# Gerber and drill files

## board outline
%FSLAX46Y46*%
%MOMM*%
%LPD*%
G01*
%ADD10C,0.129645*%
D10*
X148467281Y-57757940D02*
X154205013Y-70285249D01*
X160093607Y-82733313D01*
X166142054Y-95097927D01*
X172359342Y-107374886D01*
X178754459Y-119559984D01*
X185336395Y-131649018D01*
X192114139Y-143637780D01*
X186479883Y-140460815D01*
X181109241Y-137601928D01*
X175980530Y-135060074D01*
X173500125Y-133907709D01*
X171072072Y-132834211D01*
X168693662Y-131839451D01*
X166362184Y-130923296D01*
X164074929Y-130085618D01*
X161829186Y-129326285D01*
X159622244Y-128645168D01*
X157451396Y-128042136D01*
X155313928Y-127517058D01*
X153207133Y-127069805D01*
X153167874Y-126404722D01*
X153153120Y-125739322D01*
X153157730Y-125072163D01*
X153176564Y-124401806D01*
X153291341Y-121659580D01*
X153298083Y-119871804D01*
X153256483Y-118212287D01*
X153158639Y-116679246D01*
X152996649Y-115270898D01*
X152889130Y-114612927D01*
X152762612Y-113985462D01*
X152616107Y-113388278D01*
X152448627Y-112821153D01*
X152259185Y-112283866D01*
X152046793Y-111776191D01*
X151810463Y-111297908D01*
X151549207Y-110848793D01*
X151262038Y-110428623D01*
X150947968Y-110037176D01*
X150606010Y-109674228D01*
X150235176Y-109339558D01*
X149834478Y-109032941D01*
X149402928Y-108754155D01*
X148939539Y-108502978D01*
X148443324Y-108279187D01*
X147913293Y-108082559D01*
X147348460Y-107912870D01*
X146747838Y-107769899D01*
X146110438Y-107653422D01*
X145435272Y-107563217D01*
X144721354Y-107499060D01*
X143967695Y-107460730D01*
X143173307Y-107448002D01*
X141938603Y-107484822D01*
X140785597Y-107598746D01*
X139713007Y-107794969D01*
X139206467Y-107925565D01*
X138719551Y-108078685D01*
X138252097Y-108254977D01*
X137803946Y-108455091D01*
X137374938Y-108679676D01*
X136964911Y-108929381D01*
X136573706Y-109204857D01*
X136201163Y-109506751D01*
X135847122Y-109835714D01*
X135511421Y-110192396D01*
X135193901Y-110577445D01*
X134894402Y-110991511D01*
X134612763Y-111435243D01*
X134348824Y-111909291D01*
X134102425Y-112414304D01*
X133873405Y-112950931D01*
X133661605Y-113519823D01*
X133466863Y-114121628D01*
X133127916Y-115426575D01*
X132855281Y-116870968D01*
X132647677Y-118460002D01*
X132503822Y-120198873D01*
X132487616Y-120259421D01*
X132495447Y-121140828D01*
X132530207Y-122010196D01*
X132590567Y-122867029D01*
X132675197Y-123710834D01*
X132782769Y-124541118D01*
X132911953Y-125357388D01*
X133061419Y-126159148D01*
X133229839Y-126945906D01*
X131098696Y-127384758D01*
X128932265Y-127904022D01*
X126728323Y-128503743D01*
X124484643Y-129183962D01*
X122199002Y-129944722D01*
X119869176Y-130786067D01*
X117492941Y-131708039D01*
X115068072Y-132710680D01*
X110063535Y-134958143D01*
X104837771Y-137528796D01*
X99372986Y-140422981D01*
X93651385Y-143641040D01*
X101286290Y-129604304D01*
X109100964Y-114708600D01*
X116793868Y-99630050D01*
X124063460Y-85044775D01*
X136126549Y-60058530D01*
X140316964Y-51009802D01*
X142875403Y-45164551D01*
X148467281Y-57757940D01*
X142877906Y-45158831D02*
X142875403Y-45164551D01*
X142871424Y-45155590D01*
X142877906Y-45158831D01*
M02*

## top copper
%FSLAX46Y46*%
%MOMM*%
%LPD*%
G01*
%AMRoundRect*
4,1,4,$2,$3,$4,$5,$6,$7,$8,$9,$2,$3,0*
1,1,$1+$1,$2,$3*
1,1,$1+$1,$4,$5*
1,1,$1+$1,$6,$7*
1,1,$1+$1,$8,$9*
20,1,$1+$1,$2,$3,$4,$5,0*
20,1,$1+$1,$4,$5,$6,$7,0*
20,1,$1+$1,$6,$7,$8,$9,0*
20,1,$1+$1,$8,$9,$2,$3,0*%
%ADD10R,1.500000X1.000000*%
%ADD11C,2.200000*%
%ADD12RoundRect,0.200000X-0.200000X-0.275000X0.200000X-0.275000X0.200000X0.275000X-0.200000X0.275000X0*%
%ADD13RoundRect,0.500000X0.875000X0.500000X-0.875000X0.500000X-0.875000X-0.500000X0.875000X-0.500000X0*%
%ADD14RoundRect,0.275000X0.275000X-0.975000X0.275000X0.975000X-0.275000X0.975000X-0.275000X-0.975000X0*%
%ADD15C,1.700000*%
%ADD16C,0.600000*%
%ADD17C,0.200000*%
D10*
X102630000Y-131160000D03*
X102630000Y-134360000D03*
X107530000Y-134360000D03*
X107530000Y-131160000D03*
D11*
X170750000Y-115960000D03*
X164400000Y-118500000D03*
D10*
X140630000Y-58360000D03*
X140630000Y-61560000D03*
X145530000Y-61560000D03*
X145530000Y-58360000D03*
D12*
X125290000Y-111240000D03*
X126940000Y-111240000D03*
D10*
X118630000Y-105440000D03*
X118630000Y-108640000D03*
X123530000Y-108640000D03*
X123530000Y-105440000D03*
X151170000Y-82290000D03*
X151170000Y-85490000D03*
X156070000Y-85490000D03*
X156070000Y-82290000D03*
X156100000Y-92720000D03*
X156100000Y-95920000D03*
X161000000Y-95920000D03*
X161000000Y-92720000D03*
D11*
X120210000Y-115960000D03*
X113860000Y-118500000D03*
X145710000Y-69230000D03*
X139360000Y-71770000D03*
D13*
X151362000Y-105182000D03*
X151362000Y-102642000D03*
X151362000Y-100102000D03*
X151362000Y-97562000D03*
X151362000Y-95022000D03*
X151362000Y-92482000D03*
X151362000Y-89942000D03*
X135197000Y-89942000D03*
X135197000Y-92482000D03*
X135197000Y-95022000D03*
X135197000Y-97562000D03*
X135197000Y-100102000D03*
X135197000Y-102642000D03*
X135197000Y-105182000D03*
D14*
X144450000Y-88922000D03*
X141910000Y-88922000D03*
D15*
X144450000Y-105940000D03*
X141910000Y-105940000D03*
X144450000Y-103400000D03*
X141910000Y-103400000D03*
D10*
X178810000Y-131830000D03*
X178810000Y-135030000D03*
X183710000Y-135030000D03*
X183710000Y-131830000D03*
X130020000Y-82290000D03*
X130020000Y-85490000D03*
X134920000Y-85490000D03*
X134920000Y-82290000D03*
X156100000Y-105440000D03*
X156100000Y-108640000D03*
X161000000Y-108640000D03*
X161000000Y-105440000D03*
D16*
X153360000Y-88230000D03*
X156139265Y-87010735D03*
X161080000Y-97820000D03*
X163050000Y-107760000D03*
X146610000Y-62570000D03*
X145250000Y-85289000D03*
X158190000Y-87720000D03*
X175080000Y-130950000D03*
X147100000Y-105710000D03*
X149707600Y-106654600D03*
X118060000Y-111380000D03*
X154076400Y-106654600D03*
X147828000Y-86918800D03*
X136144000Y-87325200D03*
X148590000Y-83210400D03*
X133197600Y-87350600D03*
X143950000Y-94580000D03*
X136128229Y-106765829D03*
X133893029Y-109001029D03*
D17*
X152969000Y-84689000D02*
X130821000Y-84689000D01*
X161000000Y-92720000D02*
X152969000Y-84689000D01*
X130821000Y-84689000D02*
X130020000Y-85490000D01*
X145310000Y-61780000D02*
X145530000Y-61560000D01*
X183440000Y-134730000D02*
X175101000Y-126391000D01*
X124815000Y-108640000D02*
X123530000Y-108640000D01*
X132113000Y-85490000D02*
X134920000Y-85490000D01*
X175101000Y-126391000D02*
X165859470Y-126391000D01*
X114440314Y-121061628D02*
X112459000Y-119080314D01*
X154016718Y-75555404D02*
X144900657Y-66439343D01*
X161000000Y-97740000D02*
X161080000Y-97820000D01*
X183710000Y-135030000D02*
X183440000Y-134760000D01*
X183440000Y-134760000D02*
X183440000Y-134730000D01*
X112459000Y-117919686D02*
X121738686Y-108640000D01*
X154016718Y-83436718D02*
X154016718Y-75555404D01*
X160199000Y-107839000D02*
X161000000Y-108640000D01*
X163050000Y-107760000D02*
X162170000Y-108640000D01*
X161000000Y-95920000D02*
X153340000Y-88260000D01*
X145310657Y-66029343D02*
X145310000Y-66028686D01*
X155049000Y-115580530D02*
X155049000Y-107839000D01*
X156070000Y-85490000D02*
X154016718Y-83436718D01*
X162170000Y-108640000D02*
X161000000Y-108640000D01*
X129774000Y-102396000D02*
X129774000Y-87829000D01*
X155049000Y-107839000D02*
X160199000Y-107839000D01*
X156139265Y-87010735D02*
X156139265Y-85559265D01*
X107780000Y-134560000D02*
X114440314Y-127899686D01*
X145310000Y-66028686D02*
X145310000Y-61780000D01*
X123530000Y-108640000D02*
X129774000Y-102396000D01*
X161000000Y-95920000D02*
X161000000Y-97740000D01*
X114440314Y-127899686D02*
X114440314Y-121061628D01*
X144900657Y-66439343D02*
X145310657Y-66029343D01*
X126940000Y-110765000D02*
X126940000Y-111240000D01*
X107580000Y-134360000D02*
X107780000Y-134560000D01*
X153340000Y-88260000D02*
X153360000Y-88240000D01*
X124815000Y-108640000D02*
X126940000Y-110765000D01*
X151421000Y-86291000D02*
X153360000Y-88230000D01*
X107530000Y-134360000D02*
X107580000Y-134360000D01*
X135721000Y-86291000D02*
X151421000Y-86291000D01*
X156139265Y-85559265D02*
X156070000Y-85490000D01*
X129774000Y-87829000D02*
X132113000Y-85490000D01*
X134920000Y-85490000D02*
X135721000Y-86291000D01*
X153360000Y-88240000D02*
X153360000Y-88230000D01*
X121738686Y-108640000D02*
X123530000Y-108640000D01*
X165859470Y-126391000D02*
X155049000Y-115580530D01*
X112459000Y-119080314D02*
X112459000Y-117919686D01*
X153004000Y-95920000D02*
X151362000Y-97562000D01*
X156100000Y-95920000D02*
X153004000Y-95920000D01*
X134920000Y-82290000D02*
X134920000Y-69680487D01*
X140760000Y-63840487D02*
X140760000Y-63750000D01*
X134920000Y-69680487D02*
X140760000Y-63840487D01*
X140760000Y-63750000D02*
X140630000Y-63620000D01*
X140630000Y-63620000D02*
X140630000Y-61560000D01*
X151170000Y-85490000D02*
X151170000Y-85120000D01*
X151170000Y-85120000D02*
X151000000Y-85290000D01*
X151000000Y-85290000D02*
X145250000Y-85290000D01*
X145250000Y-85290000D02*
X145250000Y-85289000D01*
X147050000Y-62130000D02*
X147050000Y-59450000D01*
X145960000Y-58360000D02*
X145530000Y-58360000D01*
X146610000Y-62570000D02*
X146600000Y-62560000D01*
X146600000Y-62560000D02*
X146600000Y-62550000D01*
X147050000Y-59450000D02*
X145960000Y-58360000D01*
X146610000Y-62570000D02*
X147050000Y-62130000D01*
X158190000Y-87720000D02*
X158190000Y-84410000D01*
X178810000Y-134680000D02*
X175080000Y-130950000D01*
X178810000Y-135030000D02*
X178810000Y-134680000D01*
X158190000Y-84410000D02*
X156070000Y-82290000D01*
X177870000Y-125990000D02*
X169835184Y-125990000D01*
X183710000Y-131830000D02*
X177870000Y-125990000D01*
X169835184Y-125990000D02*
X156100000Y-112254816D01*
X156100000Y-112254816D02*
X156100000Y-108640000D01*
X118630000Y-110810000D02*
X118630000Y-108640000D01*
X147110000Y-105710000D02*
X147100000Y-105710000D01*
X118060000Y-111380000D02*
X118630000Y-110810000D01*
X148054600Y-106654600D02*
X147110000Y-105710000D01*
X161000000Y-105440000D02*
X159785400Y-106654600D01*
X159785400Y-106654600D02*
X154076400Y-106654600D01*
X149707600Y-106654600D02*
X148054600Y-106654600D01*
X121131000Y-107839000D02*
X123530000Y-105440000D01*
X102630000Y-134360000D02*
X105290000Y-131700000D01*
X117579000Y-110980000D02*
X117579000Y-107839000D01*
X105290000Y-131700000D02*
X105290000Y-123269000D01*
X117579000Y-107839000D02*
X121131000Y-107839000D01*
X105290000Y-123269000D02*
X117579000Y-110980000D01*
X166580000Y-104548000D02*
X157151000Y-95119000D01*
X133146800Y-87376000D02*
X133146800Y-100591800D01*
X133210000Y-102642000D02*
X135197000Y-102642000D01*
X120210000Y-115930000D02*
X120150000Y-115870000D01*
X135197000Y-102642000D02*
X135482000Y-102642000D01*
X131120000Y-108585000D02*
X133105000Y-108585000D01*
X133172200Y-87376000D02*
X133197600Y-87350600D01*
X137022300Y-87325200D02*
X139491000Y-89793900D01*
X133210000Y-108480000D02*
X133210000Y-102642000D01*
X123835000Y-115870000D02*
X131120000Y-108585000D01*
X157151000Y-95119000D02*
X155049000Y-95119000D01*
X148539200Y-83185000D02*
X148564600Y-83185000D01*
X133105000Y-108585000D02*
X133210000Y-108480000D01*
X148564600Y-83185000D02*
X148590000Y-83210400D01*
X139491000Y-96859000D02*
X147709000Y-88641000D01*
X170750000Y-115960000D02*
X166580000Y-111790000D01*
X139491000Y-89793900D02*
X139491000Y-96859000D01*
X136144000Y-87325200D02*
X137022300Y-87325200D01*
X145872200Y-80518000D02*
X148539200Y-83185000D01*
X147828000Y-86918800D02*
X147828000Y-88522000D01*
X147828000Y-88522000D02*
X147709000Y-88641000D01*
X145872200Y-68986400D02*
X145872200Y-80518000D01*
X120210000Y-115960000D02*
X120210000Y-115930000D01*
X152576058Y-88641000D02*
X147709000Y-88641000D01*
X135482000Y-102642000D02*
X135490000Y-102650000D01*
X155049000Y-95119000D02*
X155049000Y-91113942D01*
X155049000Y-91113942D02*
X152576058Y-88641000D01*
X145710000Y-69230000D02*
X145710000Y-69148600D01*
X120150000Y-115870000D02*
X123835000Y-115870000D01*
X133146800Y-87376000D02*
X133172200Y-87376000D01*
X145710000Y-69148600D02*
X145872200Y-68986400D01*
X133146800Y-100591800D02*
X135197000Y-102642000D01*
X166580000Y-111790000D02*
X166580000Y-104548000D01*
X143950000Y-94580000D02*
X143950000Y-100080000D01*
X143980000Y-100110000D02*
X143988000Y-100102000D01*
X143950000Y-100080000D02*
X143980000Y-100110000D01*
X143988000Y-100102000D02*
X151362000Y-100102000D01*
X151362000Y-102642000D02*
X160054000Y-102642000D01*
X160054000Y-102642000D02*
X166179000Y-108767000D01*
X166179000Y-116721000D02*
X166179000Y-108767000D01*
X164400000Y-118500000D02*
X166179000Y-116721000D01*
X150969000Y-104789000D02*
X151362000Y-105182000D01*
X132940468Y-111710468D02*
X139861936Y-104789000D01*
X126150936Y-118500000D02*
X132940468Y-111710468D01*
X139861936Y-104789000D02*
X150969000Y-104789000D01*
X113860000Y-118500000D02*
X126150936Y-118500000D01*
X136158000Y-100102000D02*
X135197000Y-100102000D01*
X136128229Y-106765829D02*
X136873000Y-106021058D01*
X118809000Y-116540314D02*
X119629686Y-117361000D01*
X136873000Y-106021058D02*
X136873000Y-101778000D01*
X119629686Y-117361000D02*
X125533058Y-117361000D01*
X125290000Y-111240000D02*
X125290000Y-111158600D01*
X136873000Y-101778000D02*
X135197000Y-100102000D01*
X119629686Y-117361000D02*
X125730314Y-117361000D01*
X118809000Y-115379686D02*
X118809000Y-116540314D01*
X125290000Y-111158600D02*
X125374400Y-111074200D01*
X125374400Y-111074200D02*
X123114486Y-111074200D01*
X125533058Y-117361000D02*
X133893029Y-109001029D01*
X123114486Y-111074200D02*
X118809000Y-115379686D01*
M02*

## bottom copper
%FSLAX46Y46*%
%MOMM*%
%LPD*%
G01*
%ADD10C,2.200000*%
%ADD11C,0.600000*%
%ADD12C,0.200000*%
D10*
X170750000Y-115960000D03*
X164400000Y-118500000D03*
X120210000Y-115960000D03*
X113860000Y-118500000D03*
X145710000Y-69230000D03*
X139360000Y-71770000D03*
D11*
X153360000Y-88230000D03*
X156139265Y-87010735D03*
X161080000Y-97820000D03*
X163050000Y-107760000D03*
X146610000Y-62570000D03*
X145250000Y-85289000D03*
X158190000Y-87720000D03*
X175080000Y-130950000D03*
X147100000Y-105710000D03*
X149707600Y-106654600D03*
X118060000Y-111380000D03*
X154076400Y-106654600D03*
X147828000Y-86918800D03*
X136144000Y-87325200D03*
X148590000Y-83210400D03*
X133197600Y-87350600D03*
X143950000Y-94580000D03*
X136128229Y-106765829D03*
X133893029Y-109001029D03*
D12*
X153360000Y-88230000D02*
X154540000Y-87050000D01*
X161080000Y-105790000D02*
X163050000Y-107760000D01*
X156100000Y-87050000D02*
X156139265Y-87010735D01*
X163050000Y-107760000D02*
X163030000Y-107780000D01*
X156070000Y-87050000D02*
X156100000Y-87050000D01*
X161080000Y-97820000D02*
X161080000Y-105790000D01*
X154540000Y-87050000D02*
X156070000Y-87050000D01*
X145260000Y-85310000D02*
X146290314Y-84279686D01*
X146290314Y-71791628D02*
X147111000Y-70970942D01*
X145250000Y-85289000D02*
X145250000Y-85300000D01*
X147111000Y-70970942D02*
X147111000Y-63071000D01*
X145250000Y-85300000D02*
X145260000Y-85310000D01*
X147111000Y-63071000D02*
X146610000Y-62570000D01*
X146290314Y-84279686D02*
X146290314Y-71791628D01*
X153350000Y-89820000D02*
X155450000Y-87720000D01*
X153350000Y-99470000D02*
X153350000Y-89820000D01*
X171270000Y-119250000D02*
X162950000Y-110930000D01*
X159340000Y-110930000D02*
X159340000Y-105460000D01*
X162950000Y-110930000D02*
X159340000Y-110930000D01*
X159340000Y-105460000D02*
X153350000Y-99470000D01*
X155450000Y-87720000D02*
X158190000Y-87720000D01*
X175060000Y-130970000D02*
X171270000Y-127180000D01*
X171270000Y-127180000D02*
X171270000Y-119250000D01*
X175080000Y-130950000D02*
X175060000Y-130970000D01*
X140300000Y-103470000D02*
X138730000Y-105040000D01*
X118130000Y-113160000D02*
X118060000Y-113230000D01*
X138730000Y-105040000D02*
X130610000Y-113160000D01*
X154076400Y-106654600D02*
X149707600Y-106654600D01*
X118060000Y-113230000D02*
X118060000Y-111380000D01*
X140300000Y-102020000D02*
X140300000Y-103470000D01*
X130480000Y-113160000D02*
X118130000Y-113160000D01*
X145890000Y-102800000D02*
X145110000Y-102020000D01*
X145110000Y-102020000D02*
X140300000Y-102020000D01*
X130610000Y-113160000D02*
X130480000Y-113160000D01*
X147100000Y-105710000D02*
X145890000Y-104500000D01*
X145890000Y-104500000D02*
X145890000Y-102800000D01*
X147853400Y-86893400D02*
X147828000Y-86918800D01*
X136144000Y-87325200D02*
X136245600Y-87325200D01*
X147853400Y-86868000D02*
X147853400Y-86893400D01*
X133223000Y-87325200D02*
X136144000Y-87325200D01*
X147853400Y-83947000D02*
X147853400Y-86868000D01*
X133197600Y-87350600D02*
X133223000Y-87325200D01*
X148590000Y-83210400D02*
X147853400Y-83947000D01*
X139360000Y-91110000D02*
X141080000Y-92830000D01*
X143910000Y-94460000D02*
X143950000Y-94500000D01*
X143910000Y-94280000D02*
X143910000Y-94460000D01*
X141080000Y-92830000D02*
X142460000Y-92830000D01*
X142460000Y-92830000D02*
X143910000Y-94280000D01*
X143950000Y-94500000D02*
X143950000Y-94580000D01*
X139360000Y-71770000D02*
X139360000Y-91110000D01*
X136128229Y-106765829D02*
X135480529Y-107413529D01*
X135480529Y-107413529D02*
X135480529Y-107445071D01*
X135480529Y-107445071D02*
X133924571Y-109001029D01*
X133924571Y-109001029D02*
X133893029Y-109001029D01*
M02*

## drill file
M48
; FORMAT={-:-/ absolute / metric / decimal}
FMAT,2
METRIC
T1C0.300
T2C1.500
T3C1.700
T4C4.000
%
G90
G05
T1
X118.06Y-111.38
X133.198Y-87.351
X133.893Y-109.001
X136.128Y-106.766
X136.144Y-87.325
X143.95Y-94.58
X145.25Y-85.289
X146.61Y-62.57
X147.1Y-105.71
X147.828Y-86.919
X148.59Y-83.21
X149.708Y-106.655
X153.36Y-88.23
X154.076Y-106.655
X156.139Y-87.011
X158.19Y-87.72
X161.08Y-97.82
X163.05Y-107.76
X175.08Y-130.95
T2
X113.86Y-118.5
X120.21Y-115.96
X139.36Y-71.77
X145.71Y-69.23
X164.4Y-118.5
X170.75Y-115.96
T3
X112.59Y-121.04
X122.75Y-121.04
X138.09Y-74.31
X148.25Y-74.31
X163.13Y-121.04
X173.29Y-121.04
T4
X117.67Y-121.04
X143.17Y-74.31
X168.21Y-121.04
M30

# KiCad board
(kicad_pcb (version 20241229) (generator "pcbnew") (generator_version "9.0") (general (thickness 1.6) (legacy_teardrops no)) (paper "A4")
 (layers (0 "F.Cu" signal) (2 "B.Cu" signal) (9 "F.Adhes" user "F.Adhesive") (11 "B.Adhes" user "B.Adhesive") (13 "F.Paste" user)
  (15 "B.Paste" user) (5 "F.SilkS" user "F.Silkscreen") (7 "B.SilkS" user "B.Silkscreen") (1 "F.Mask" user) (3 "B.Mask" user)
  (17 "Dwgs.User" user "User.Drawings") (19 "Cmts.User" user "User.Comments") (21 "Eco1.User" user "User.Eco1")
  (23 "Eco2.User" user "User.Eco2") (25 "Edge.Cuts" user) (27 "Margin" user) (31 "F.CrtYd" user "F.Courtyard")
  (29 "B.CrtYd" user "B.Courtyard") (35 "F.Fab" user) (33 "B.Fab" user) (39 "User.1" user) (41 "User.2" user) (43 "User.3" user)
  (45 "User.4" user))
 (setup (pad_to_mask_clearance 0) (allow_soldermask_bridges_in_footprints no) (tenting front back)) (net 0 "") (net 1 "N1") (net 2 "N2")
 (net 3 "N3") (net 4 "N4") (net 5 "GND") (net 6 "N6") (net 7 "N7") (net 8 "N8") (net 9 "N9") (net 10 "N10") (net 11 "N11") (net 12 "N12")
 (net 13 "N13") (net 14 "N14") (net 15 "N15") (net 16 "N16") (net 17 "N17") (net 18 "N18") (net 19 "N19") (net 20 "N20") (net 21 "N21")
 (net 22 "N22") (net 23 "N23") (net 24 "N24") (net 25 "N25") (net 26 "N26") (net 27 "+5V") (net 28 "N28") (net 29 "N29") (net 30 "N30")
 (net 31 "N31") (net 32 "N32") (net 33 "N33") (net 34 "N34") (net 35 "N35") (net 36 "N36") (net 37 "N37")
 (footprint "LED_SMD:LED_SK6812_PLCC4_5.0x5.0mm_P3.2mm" (layer "F.Cu") (at 105.08 132.76)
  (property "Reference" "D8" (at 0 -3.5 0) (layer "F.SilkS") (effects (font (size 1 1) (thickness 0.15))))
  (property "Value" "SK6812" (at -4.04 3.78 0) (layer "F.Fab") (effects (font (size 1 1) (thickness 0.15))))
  (pad "1" smd rect (at -2.45 -1.6 180) (size 1.5 1) (layers "F.Cu" "F.Mask" "F.Paste") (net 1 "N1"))
  (pad "2" smd rect (at -2.45 1.6 180) (size 1.5 1) (layers "F.Cu" "F.Mask" "F.Paste") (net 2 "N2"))
  (pad "3" smd rect (at 2.45 1.6 180) (size 1.5 1) (layers "F.Cu" "F.Mask" "F.Paste") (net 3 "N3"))
  (pad "4" smd rect (at 2.45 -1.6 180) (size 1.5 1) (layers "F.Cu" "F.Mask" "F.Paste") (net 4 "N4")))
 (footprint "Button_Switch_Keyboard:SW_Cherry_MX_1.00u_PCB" (layer "F.Cu") (at 170.75 115.96)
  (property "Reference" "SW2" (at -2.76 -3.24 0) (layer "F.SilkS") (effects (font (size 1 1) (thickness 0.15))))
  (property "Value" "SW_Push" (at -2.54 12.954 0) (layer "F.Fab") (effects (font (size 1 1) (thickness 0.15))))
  (pad "" np_thru_hole circle (at -7.62 5.08) (size 1.7 1.7) (drill 1.7) (layers "*.Cu" "*.Mask"))
  (pad "" np_thru_hole circle (at -2.54 5.08) (size 4 4) (drill 4) (layers "*.Cu" "*.Mask"))
  (pad "" np_thru_hole circle (at 2.54 5.08) (size 1.7 1.7) (drill 1.7) (layers "*.Cu" "*.Mask"))
  (pad "1" thru_hole circle (at 0 0) (size 2.2 2.2) (drill 1.5) (layers "*.Cu" "*.Mask") (remove_unused_layers no) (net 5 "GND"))
  (pad "2" thru_hole circle (at -6.35 2.54) (size 2.2 2.2) (drill 1.5) (layers "*.Cu" "*.Mask") (remove_unused_layers no) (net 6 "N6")))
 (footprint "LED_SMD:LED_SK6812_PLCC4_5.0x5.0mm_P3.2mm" (layer "F.Cu") (at 143.08 59.96)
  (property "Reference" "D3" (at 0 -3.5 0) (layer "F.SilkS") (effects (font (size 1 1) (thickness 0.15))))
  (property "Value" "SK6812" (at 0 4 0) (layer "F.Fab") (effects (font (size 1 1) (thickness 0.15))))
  (pad "1" smd rect (at -2.45 -1.6 180) (size 1.5 1) (layers "F.Cu" "F.Mask" "F.Paste") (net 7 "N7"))
  (pad "2" smd rect (at -2.45 1.6 180) (size 1.5 1) (layers "F.Cu" "F.Mask" "F.Paste") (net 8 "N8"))
  (pad "3" smd rect (at 2.45 1.6 180) (size 1.5 1) (layers "F.Cu" "F.Mask" "F.Paste") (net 3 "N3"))
  (pad "4" smd rect (at 2.45 -1.6 180) (size 1.5 1) (layers "F.Cu" "F.Mask" "F.Paste") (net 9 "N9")))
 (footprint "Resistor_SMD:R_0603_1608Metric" (layer "F.Cu") (at 126.115 111.24)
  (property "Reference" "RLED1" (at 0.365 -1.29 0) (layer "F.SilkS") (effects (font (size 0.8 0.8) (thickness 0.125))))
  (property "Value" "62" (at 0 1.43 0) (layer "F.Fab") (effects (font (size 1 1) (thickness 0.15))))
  (pad "1" smd roundrect (at -0.825 0) (size 0.8 0.95) (layers "F.Cu" "F.Mask" "F.Paste") (roundrect_rratio 0.25) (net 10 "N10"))
  (pad "2" smd roundrect (at 0.825 0) (size 0.8 0.95) (layers "F.Cu" "F.Mask" "F.Paste") (roundrect_rratio 0.25) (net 3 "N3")))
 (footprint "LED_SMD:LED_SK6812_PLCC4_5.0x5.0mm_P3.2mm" (layer "F.Cu") (at 121.08 107.04)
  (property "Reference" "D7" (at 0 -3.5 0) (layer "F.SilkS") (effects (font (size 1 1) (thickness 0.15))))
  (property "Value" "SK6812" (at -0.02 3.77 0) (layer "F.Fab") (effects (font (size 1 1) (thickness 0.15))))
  (pad "1" smd rect (at -2.45 -1.6 180) (size 1.5 1) (layers "F.Cu" "F.Mask" "F.Paste") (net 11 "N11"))
  (pad "2" smd rect (at -2.45 1.6 180) (size 1.5 1) (layers "F.Cu" "F.Mask" "F.Paste") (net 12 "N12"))
  (pad "3" smd rect (at 2.45 1.6 180) (size 1.5 1) (layers "F.Cu" "F.Mask" "F.Paste") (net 3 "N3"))
  (pad "4" smd rect (at 2.45 -1.6 180) (size 1.5 1) (layers "F.Cu" "F.Mask" "F.Paste") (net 2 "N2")))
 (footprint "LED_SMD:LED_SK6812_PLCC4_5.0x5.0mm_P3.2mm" (layer "F.Cu") (at 153.62 83.89)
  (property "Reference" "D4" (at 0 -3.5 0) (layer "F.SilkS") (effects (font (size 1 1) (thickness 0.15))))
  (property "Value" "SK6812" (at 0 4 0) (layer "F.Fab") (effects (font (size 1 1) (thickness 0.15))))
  (pad "1" smd rect (at -2.45 -1.6 180) (size 1.5 1) (layers "F.Cu" "F.Mask" "F.Paste") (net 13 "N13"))
  (pad "2" smd rect (at -2.45 1.6 180) (size 1.5 1) (layers "F.Cu" "F.Mask" "F.Paste") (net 9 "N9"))
  (pad "3" smd rect (at 2.45 1.6 180) (size 1.5 1) (layers "F.Cu" "F.Mask" "F.Paste") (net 3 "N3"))
  (pad "4" smd rect (at 2.45 -1.6 180) (size 1.5 1) (layers "F.Cu" "F.Mask" "F.Paste") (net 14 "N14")))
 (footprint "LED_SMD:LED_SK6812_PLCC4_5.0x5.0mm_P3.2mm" (layer "F.Cu") (at 158.55 94.32)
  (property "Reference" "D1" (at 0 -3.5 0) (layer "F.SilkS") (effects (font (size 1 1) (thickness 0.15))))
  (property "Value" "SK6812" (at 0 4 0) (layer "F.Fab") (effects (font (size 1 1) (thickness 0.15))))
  (pad "1" smd rect (at -2.45 -1.6 180) (size 1.5 1) (layers "F.Cu" "F.Mask" "F.Paste") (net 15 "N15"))
  (pad "2" smd rect (at -2.45 1.6 180) (size 1.5 1) (layers "F.Cu" "F.Mask" "F.Paste") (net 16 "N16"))
  (pad "3" smd rect (at 2.45 1.6 180) (size 1.5 1) (layers "F.Cu" "F.Mask" "F.Paste") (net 3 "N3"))
  (pad "4" smd rect (at 2.45 -1.6 180) (size 1.5 1) (layers "F.Cu" "F.Mask" "F.Paste") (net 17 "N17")))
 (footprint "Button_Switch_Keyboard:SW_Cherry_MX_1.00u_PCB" (layer "F.Cu") (at 120.21 115.96)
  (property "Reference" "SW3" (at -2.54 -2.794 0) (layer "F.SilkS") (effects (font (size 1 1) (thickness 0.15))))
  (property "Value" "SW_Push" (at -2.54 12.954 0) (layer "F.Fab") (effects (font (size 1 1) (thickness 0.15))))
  (pad "" np_thru_hole circle (at -7.62 5.08) (size 1.7 1.7) (drill 1.7) (layers "*.Cu" "*.Mask"))
  (pad "" np_thru_hole circle (at -2.54 5.08) (size 4 4) (drill 4) (layers "*.Cu" "*.Mask"))
  (pad "" np_thru_hole circle (at 2.54 5.08) (size 1.7 1.7) (drill 1.7) (layers "*.Cu" "*.Mask"))
  (pad "1" thru_hole circle (at 0 0) (size 2.2 2.2) (drill 1.5) (layers "*.Cu" "*.Mask") (remove_unused_layers no) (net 5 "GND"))
  (pad "2" thru_hole circle (at -6.35 2.54) (size 2.2 2.2) (drill 1.5) (layers "*.Cu" "*.Mask") (remove_unused_layers no) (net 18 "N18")))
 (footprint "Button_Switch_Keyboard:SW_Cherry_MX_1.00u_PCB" (layer "F.Cu") (at 145.71 69.23)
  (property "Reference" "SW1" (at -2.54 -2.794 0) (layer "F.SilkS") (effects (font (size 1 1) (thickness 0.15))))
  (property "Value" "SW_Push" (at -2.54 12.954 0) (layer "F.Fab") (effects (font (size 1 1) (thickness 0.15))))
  (pad "" np_thru_hole circle (at -7.62 5.08) (size 1.7 1.7) (drill 1.7) (layers "*.Cu" "*.Mask"))
  (pad "" np_thru_hole circle (at -2.54 5.08) (size 4 4) (drill 4) (layers "*.Cu" "*.Mask"))
  (pad "" np_thru_hole circle (at 2.54 5.08) (size 1.7 1.7) (drill 1.7) (layers "*.Cu" "*.Mask"))
  (pad "1" thru_hole circle (at 0 0) (size 2.2 2.2) (drill 1.5) (layers "*.Cu" "*.Mask") (remove_unused_layers no) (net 5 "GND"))
  (pad "2" thru_hole circle (at -6.35 2.54) (size 2.2 2.2) (drill 1.5) (layers "*.Cu" "*.Mask") (remove_unused_layers no) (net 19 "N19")))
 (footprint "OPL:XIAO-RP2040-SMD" (layer "F.Cu") (at 143.362 97.562 180)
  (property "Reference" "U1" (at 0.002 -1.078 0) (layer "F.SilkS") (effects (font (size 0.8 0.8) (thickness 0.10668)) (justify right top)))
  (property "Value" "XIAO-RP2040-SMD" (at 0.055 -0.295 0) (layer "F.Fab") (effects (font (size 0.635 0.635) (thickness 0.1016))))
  (pad "1" smd roundrect (at -8 -7.62 180) (size 2.75 2) (layers "F.Cu" "F.Mask" "F.Paste") (roundrect_rratio 0.25) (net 18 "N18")
   (solder_mask_margin 0.0508) (thermal_bridge_angle 45))
  (pad "2" smd roundrect (at -8 -5.08 180) (size 2.75 2) (layers "F.Cu" "F.Mask" "F.Paste") (roundrect_rratio 0.25) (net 6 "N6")
   (solder_mask_margin 0.0508) (thermal_bridge_angle 45))
  (pad "3" smd roundrect (at -8 -2.54 180) (size 2.75 2) (layers "F.Cu" "F.Mask" "F.Paste") (roundrect_rratio 0.25) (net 19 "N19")
   (solder_mask_margin 0.0508) (thermal_bridge_angle 45))
  (pad "4" smd roundrect (at -8 0 180) (size 2.75 2) (layers "F.Cu" "F.Mask" "F.Paste") (roundrect_rratio 0.25) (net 16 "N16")
   (solder_mask_margin 0.0508) (thermal_bridge_angle 45))
  (pad "5" smd roundrect (at -8 2.54 180) (size 2.75 2) (layers "F.Cu" "F.Mask" "F.Paste") (roundrect_rratio 0.25) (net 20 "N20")
   (solder_mask_margin 0.0508) (thermal_bridge_angle 45))
  (pad "6" smd roundrect (at -8 5.08 180) (size 2.75 2) (layers "F.Cu" "F.Mask" "F.Paste") (roundrect_rratio 0.25) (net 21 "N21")
   (solder_mask_margin 0.0508) (thermal_bridge_angle 45))
  (pad "7" smd roundrect (at -8 7.62 180) (size 2.75 2) (layers "F.Cu" "F.Mask" "F.Paste") (roundrect_rratio 0.25) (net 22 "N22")
   (solder_mask_margin 0.0508) (thermal_bridge_angle 45))
  (pad "8" smd roundrect (at 8.165 7.62 180) (size 2.75 2) (layers "F.Cu" "F.Mask" "F.Paste") (roundrect_rratio 0.25) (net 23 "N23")
   (solder_mask_margin 0.0508) (thermal_bridge_angle 45))
  (pad "9" smd roundrect (at 8.165 5.08 180) (size 2.75 2) (layers "F.Cu" "F.Mask" "F.Paste") (roundrect_rratio 0.25) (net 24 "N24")
   (solder_mask_margin 0.0508) (thermal_bridge_angle 45))
  (pad "10" smd roundrect (at 8.165 2.54 180) (size 2.75 2) (layers "F.Cu" "F.Mask" "F.Paste") (roundrect_rratio 0.25) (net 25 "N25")
   (solder_mask_margin 0.0508) (thermal_bridge_angle 45))
  (pad "11" smd roundrect (at 8.165 0 180) (size 2.75 2) (layers "F.Cu" "F.Mask" "F.Paste") (roundrect_rratio 0.25) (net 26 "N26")
   (solder_mask_margin 0.0508) (thermal_bridge_angle 45))
  (pad "12" smd roundrect (at 8.165 -2.54 180) (size 2.75 2) (layers "F.Cu" "F.Mask" "F.Paste") (roundrect_rratio 0.25) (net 10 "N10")
   (solder_mask_margin 0.0508) (thermal_bridge_angle 45))
  (pad "13" smd roundrect (at 8.165 -5.08 180) (size 2.75 2) (layers "F.Cu" "F.Mask" "F.Paste") (roundrect_rratio 0.25) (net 5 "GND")
   (solder_mask_margin 0.0508) (thermal_bridge_angle 45))
  (pad "14" smd roundrect (at 8.165 -7.62 180) (size 2.75 2) (layers "F.Cu" "F.Mask" "F.Paste") (roundrect_rratio 0.25) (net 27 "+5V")
   (solder_mask_margin 0.0508) (thermal_bridge_angle 45))
  (pad "15" smd roundrect (at -1.088 8.64 90) (size 2.5 1.1) (layers "F.Cu" "F.Mask" "F.Paste") (roundrect_rratio 0.25) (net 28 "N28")
   (thermal_bridge_angle 45))
  (pad "16" smd roundrect (at 1.452 8.64 90) (size 2.5 1.1) (layers "F.Cu" "F.Mask" "F.Paste") (roundrect_rratio 0.25) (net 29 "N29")
   (thermal_bridge_angle 45))
  (pad "17" smd circle (at -1.088 -8.378 180) (size 1.7 1.7) (layers "F.Cu" "F.Mask" "F.Paste") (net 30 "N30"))
  (pad "18" smd circle (at 1.452 -8.378 180) (size 1.7 1.7) (layers "F.Cu" "F.Mask" "F.Paste") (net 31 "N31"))
  (pad "19" smd circle (at -1.088 -5.838 180) (size 1.7 1.7) (layers "F.Cu" "F.Mask" "F.Paste") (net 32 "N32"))
  (pad "20" smd circle (at 1.452 -5.838 180) (size 1.7 1.7) (layers "F.Cu" "F.Mask" "F.Paste") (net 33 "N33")))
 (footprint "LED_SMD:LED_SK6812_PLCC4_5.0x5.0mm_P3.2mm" (layer "F.Cu") (at 181.26 133.43)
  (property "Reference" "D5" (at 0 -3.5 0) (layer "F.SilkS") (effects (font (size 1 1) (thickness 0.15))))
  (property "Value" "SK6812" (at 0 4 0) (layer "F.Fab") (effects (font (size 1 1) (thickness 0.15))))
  (pad "1" smd rect (at -2.45 -1.6 180) (size 1.5 1) (layers "F.Cu" "F.Mask" "F.Paste") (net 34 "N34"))
  (pad "2" smd rect (at -2.45 1.6 180) (size 1.5 1) (layers "F.Cu" "F.Mask" "F.Paste") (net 14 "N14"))
  (pad "3" smd rect (at 2.45 1.6 180) (size 1.5 1) (layers "F.Cu" "F.Mask" "F.Paste") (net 3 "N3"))
  (pad "4" smd rect (at 2.45 -1.6 180) (size 1.5 1) (layers "F.Cu" "F.Mask" "F.Paste") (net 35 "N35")))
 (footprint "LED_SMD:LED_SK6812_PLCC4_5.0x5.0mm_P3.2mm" (layer "F.Cu") (at 132.47 83.89)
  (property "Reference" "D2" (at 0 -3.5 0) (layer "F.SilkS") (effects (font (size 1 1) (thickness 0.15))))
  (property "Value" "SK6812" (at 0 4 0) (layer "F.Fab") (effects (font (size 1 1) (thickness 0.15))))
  (pad "1" smd rect (at -2.45 -1.6 180) (size 1.5 1) (layers "F.Cu" "F.Mask" "F.Paste") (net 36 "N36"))
  (pad "2" smd rect (at -2.45 1.6 180) (size 1.5 1) (layers "F.Cu" "F.Mask" "F.Paste") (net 17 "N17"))
  (pad "3" smd rect (at 2.45 1.6 180) (size 1.5 1) (layers "F.Cu" "F.Mask" "F.Paste") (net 3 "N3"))
  (pad "4" smd rect (at 2.45 -1.6 180) (size 1.5 1) (layers "F.Cu" "F.Mask" "F.Paste") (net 8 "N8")))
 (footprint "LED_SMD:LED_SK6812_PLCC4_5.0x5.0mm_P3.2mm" (layer "F.Cu") (at 158.55 107.04)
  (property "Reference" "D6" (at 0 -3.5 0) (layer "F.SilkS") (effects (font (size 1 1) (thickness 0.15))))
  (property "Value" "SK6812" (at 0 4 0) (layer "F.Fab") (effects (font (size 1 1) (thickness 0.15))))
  (pad "1" smd rect (at -2.45 -1.6 180) (size 1.5 1) (layers "F.Cu" "F.Mask" "F.Paste") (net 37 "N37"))
  (pad "2" smd rect (at -2.45 1.6 180) (size 1.5 1) (layers "F.Cu" "F.Mask" "F.Paste") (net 35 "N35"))
  (pad "3" smd rect (at 2.45 1.6 180) (size 1.5 1) (layers "F.Cu" "F.Mask" "F.Paste") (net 3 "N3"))
  (pad "4" smd rect (at 2.45 -1.6 180) (size 1.5 1) (layers "F.Cu" "F.Mask" "F.Paste") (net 12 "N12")))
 (gr_poly
  (pts (xy 148.467281 57.75794) (xy 154.205013 70.285249) (xy 160.093607 82.733313) (xy 166.142054 95.097927) (xy 172.359342 107.374886)
   (xy 178.754459 119.559984) (xy 185.336395 131.649018) (xy 192.114139 143.63778) (xy 186.479883 140.460815) (xy 181.109241 137.601928)
   (xy 175.98053 135.060074) (xy 173.500125 133.907709) (xy 171.072072 132.834211) (xy 168.693662 131.839451) (xy 166.362184 130.923296)
   (xy 164.074929 130.085618) (xy 161.829186 129.326285) (xy 159.622244 128.645168) (xy 157.451396 128.042136) (xy 155.313928 127.517058)
   (xy 153.207133 127.069805) (xy 153.167874 126.404722) (xy 153.15312 125.739322) (xy 153.15773 125.072163) (xy 153.176564 124.401806)
   (xy 153.291341 121.65958) (xy 153.298083 119.871804) (xy 153.256483 118.212287) (xy 153.158639 116.679246) (xy 152.996649 115.270898)
   (xy 152.88913 114.612927) (xy 152.762612 113.985462) (xy 152.616107 113.388278) (xy 152.448627 112.821153) (xy 152.259185 112.283866)
   (xy 152.046793 111.776191) (xy 151.810463 111.297908) (xy 151.549207 110.848793) (xy 151.262038 110.428623) (xy 150.947968 110.037176)
   (xy 150.60601 109.674228) (xy 150.235176 109.339558) (xy 149.834478 109.032941) (xy 149.402928 108.754155) (xy 148.939539 108.502978)
   (xy 148.443324 108.279187) (xy 147.913293 108.082559) (xy 147.34846 107.91287) (xy 146.747838 107.769899) (xy 146.110438 107.653422)
   (xy 145.435272 107.563217) (xy 144.721354 107.49906) (xy 143.967695 107.46073) (xy 143.173307 107.448002) (xy 141.938603 107.484822)
   (xy 140.785597 107.598746) (xy 139.713007 107.794969) (xy 139.206467 107.925565) (xy 138.719551 108.078685) (xy 138.252097 108.254977)
   (xy 137.803946 108.455091) (xy 137.374938 108.679676) (xy 136.964911 108.929381) (xy 136.573706 109.204857) (xy 136.201163 109.506751)
   (xy 135.847122 109.835714) (xy 135.511421 110.192396) (xy 135.193901 110.577445) (xy 134.894402 110.991511) (xy 134.612763 111.435243)
   (xy 134.348824 111.909291) (xy 134.102425 112.414304) (xy 133.873405 112.950931) (xy 133.661605 113.519823) (xy 133.466863 114.121628)
   (xy 133.127916 115.426575) (xy 132.855281 116.870968) (xy 132.647677 118.460002) (xy 132.503822 120.198873) (xy 132.487616 120.259421)
   (xy 132.495447 121.140828) (xy 132.530207 122.010196) (xy 132.590567 122.867029) (xy 132.675197 123.710834) (xy 132.782769 124.541118)
   (xy 132.911953 125.357388) (xy 133.061419 126.159148) (xy 133.229839 126.945906) (xy 131.098696 127.384758) (xy 128.932265 127.904022)
   (xy 126.728323 128.503743) (xy 124.484643 129.183962) (xy 122.199002 129.944722) (xy 119.869176 130.786067) (xy 117.492941 131.708039)
   (xy 115.068072 132.71068) (xy 110.063535 134.958143) (xy 104.837771 137.528796) (xy 99.372986 140.422981) (xy 93.651385 143.64104)
   (xy 101.28629 129.604304) (xy 109.100964 114.7086) (xy 116.793868 99.63005) (xy 124.06346 85.044775) (xy 136.126549 60.05853)
   (xy 140.316964 51.009802) (xy 142.875403 45.164551))
  (stroke (width 0.129645) (type solid)) (fill no) (layer "Edge.Cuts"))
 (gr_poly
  (pts (xy 142.877906 45.158831) (xy 142.875403 45.164551) (xy 142.871424 45.15559)) (stroke (width 0.129645) (type solid)) (fill no)
  (layer "Edge.Cuts"))
 (segment (start 152.969 84.689) (end 130.821 84.689) (width 0.2) (layer "F.Cu") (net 17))
 (segment (start 161 92.72) (end 152.969 84.689) (width 0.2) (layer "F.Cu") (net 17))
 (segment (start 130.821 84.689) (end 130.02 85.49) (width 0.2) (layer "F.Cu") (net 17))
 (segment (start 145.31 61.78) (end 145.53 61.56) (width 0.2) (layer "F.Cu") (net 3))
 (segment (start 183.44 134.73) (end 175.101 126.391) (width 0.2) (layer "F.Cu") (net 3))
 (segment (start 124.815 108.64) (end 123.53 108.64) (width 0.2) (layer "F.Cu") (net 3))
 (segment (start 132.113 85.49) (end 134.92 85.49) (width 0.2) (layer "F.Cu") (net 3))
 (segment (start 175.101 126.391) (end 165.85947 126.391) (width 0.2) (layer "F.Cu") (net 3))
 (segment (start 114.440314 121.061628) (end 112.459 119.080314) (width 0.2) (layer "F.Cu") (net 3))
 (segment (start 154.016718 75.555404) (end 144.900657 66.439343) (width 0.2) (layer "F.Cu") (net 3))
 (segment (start 161 97.74) (end 161.08 97.82) (width 0.2) (layer "F.Cu") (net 3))
 (segment (start 183.71 135.03) (end 183.44 134.76) (width 0.2) (layer "F.Cu") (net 3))
 (segment (start 183.44 134.76) (end 183.44 134.73) (width 0.2) (layer "F.Cu") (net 3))
 (segment (start 112.459 117.919686) (end 121.738686 108.64) (width 0.2) (layer "F.Cu") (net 3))
 (segment (start 154.016718 83.436718) (end 154.016718 75.555404) (width 0.2) (layer "F.Cu") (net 3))
 (segment (start 160.199 107.839) (end 161 108.64) (width 0.2) (layer "F.Cu") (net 3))
 (segment (start 163.05 107.76) (end 162.17 108.64) (width 0.2) (layer "F.Cu") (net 3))
 (segment (start 161 95.92) (end 153.34 88.26) (width 0.2) (layer "F.Cu") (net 3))
 (segment (start 145.310657 66.029343) (end 145.31 66.028686) (width 0.2) (layer "F.Cu") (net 3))
 (segment (start 155.049 115.58053) (end 155.049 107.839) (width 0.2) (layer "F.Cu") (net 3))
 (segment (start 156.07 85.49) (end 154.016718 83.436718) (width 0.2) (layer "F.Cu") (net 3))
 (segment (start 162.17 108.64) (end 161 108.64) (width 0.2) (layer "F.Cu") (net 3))
 (segment (start 129.774 102.396) (end 129.774 87.829) (width 0.2) (layer "F.Cu") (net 3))
 (segment (start 155.049 107.839) (end 160.199 107.839) (width 0.2) (layer "F.Cu") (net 3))
 (segment (start 156.139265 87.010735) (end 156.139265 85.559265) (width 0.2) (layer "F.Cu") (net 3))
 (segment (start 107.78 134.56) (end 114.440314 127.899686) (width 0.2) (layer "F.Cu") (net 3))
 (segment (start 145.31 66.028686) (end 145.31 61.78) (width 0.2) (layer "F.Cu") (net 3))
 (segment (start 123.53 108.64) (end 129.774 102.396) (width 0.2) (layer "F.Cu") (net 3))
 (segment (start 161 95.92) (end 161 97.74) (width 0.2) (layer "F.Cu") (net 3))
 (segment (start 114.440314 127.899686) (end 114.440314 121.061628) (width 0.2) (layer "F.Cu") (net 3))
 (segment (start 144.900657 66.439343) (end 145.310657 66.029343) (width 0.2) (layer "F.Cu") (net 3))
 (segment (start 126.94 110.765) (end 126.94 111.24) (width 0.2) (layer "F.Cu") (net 3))
 (segment (start 107.58 134.36) (end 107.78 134.56) (width 0.2) (layer "F.Cu") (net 3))
 (segment (start 153.34 88.26) (end 153.36 88.24) (width 0.2) (layer "F.Cu") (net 3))
 (segment (start 124.815 108.64) (end 126.94 110.765) (width 0.2) (layer "F.Cu") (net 3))
 (segment (start 151.421 86.291) (end 153.36 88.23) (width 0.2) (layer "F.Cu") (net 3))
 (segment (start 107.53 134.36) (end 107.58 134.36) (width 0.2) (layer "F.Cu") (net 3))
 (segment (start 135.721 86.291) (end 151.421 86.291) (width 0.2) (layer "F.Cu") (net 3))
 (segment (start 156.139265 85.559265) (end 156.07 85.49) (width 0.2) (layer "F.Cu") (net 3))
 (segment (start 129.774 87.829) (end 132.113 85.49) (width 0.2) (layer "F.Cu") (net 3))
 (segment (start 134.92 85.49) (end 135.721 86.291) (width 0.2) (layer "F.Cu") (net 3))
 (segment (start 153.36 88.24) (end 153.36 88.23) (width 0.2) (layer "F.Cu") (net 3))
 (segment (start 121.738686 108.64) (end 123.53 108.64) (width 0.2) (layer "F.Cu") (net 3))
 (segment (start 165.85947 126.391) (end 155.049 115.58053) (width 0.2) (layer "F.Cu") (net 3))
 (segment (start 112.459 119.080314) (end 112.459 117.919686) (width 0.2) (layer "F.Cu") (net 3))
 (via (at 153.36 88.23) (size 0.6) (drill 0.3) (layers "F.Cu" "B.Cu") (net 3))
 (via (at 156.139265 87.010735) (size 0.6) (drill 0.3) (layers "F.Cu" "B.Cu") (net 3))
 (via (at 161.08 97.82) (size 0.6) (drill 0.3) (layers "F.Cu" "B.Cu") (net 3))
 (via (at 163.05 107.76) (size 0.6) (drill 0.3) (layers "F.Cu" "B.Cu") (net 3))
 (segment (start 153.36 88.23) (end 154.54 87.05) (width 0.2) (layer "B.Cu") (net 3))
 (segment (start 161.08 105.79) (end 163.05 107.76) (width 0.2) (layer "B.Cu") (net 3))
 (segment (start 156.1 87.05) (end 156.139265 87.010735) (width 0.2) (layer "B.Cu") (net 3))
 (segment (start 163.05 107.76) (end 163.03 107.78) (width 0.2) (layer "B.Cu") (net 3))
 (segment (start 156.07 87.05) (end 156.1 87.05) (width 0.2) (layer "B.Cu") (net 3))
 (segment (start 161.08 97.82) (end 161.08 105.79) (width 0.2) (layer "B.Cu") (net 3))
 (segment (start 154.54 87.05) (end 156.07 87.05) (width 0.2) (layer "B.Cu") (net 3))
 (segment (start 153.004 95.92) (end 151.362 97.562) (width 0.2) (layer "F.Cu") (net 16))
 (segment (start 156.1 95.92) (end 153.004 95.92) (width 0.2) (layer "F.Cu") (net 16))
 (segment (start 134.92 82.29) (end 134.92 69.680487) (width 0.2) (layer "F.Cu") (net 8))
 (segment (start 140.76 63.840487) (end 140.76 63.75) (width 0.2) (layer "F.Cu") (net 8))
 (segment (start 134.92 69.680487) (end 140.76 63.840487) (width 0.2) (layer "F.Cu") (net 8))
 (segment (start 140.76 63.75) (end 140.63 63.62) (width 0.2) (layer "F.Cu") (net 8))
 (segment (start 140.63 63.62) (end 140.63 61.56) (width 0.2) (layer "F.Cu") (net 8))
 (segment (start 151.17 85.49) (end 151.17 85.12) (width 0.2) (layer "F.Cu") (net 9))
 (segment (start 151.17 85.12) (end 151 85.29) (width 0.2) (layer "F.Cu") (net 9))
 (segment (start 151 85.29) (end 145.25 85.29) (width 0.2) (layer "F.Cu") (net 9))
 (segment (start 145.25 85.29) (end 145.25 85.289) (width 0.2) (layer "F.Cu") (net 9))
 (segment (start 147.05 62.13) (end 147.05 59.45) (width 0.2) (layer "F.Cu") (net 9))
 (segment (start 145.96 58.36) (end 145.53 58.36) (width 0.2) (layer "F.Cu") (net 9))
 (segment (start 146.61 62.57) (end 146.6 62.56) (width 0.2) (layer "F.Cu") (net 9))
 (segment (start 146.6 62.56) (end 146.6 62.55) (width 0.2) (layer "F.Cu") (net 9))
 (segment (start 147.05 59.45) (end 145.96 58.36) (width 0.2) (layer "F.Cu") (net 9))
 (segment (start 146.61 62.57) (end 147.05 62.13) (width 0.2) (layer "F.Cu") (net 9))
 (via (at 146.61 62.57) (size 0.6) (drill 0.3) (layers "F.Cu" "B.Cu") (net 9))
 (via (at 145.25 85.289) (size 0.6) (drill 0.3) (layers "F.Cu" "B.Cu") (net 9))
 (segment (start 145.26 85.31) (end 146.290314 84.279686) (width 0.2) (layer "B.Cu") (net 9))
 (segment (start 146.290314 71.791628) (end 147.111 70.970942) (width 0.2) (layer "B.Cu") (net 9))
 (segment (start 145.25 85.289) (end 145.25 85.3) (width 0.2) (layer "B.Cu") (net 9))
 (segment (start 147.111 70.970942) (end 147.111 63.071) (width 0.2) (layer "B.Cu") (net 9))
 (segment (start 145.25 85.3) (end 145.26 85.31) (width 0.2) (layer "B.Cu") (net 9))
 (segment (start 147.111 63.071) (end 146.61 62.57) (width 0.2) (layer "B.Cu") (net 9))
 (segment (start 146.290314 84.279686) (end 146.290314 71.791628) (width 0.2) (layer "B.Cu") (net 9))
 (segment (start 158.19 87.72) (end 158.19 84.41) (width 0.2) (layer "F.Cu") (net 14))
 (segment (start 178.81 134.68) (end 175.08 130.95) (width 0.2) (layer "F.Cu") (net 14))
 (segment (start 178.81 135.03) (end 178.81 134.68) (width 0.2) (layer "F.Cu") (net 14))
 (segment (start 158.19 84.41) (end 156.07 82.29) (width 0.2) (layer "F.Cu") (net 14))
 (via (at 158.19 87.72) (size 0.6) (drill 0.3) (layers "F.Cu" "B.Cu") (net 14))
 (via (at 175.08 130.95) (size 0.6) (drill 0.3) (layers "F.Cu" "B.Cu") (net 14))
 (segment (start 153.35 89.82) (end 155.45 87.72) (width 0.2) (layer "B.Cu") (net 14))
 (segment (start 153.35 99.47) (end 153.35 89.82) (width 0.2) (layer "B.Cu") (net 14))
 (segment (start 171.27 119.25) (end 162.95 110.93) (width 0.2) (layer "B.Cu") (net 14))
 (segment (start 159.34 110.93) (end 159.34 105.46) (width 0.2) (layer "B.Cu") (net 14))
 (segment (start 162.95 110.93) (end 159.34 110.93) (width 0.2) (layer "B.Cu") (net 14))
 (segment (start 159.34 105.46) (end 153.35 99.47) (width 0.2) (layer "B.Cu") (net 14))
 (segment (start 155.45 87.72) (end 158.19 87.72) (width 0.2) (layer "B.Cu") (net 14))
 (segment (start 175.06 130.97) (end 171.27 127.18) (width 0.2) (layer "B.Cu") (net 14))
 (segment (start 171.27 127.18) (end 171.27 119.25) (width 0.2) (layer "B.Cu") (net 14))
 (segment (start 175.08 130.95) (end 175.06 130.97) (width 0.2) (layer "B.Cu") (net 14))
 (segment (start 177.87 125.99) (end 169.835184 125.99) (width 0.2) (layer "F.Cu") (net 35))
 (segment (start 183.71 131.83) (end 177.87 125.99) (width 0.2) (layer "F.Cu") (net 35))
 (segment (start 169.835184 125.99) (end 156.1 112.254816) (width 0.2) (layer "F.Cu") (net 35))
 (segment (start 156.1 112.254816) (end 156.1 108.64) (width 0.2) (layer "F.Cu") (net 35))
 (segment (start 118.63 110.81) (end 118.63 108.64) (width 0.2) (layer "F.Cu") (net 12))
 (segment (start 147.11 105.71) (end 147.1 105.71) (width 0.2) (layer "F.Cu") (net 12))
 (segment (start 118.06 111.38) (end 118.63 110.81) (width 0.2) (layer "F.Cu") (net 12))
 (segment (start 148.0546 106.6546) (end 147.11 105.71) (width 0.2) (layer "F.Cu") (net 12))
 (segment (start 161 105.44) (end 159.7854 106.6546) (width 0.2) (layer "F.Cu") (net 12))
 (segment (start 159.7854 106.6546) (end 154.0764 106.6546) (width 0.2) (layer "F.Cu") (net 12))
 (segment (start 149.7076 106.6546) (end 148.0546 106.6546) (width 0.2) (layer "F.Cu") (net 12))
 (via (at 147.1 105.71) (size 0.6) (drill 0.3) (layers "F.Cu" "B.Cu") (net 12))
 (via (at 149.7076 106.6546) (size 0.6) (drill 0.3) (layers "F.Cu" "B.Cu") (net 12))
 (via (at 118.06 111.38) (size 0.6) (drill 0.3) (layers "F.Cu" "B.Cu") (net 12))
 (via (at 154.0764 106.6546) (size 0.6) (drill 0.3) (layers "F.Cu" "B.Cu") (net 12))
 (segment (start 140.3 103.47) (end 138.73 105.04) (width 0.2) (layer "B.Cu") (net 12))
 (segment (start 118.13 113.16) (end 118.06 113.23) (width 0.2) (layer "B.Cu") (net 12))
 (segment (start 138.73 105.04) (end 130.61 113.16) (width 0.2) (layer "B.Cu") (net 12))
 (segment (start 154.0764 106.6546) (end 149.7076 106.6546) (width 0.2) (layer "B.Cu") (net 12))
 (segment (start 118.06 113.23) (end 118.06 111.38) (width 0.2) (layer "B.Cu") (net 12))
 (segment (start 140.3 102.02) (end 140.3 103.47) (width 0.2) (layer "B.Cu") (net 12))
 (segment (start 130.48 113.16) (end 118.13 113.16) (width 0.2) (layer "B.Cu") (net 12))
 (segment (start 145.89 102.8) (end 145.11 102.02) (width 0.2) (layer "B.Cu") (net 12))
 (segment (start 145.11 102.02) (end 140.3 102.02) (width 0.2) (layer "B.Cu") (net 12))
 (segment (start 130.61 113.16) (end 130.48 113.16) (width 0.2) (layer "B.Cu") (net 12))
 (segment (start 147.1 105.71) (end 145.89 104.5) (width 0.2) (layer "B.Cu") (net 12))
 (segment (start 145.89 104.5) (end 145.89 102.8) (width 0.2) (layer "B.Cu") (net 12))
 (segment (start 121.131 107.839) (end 123.53 105.44) (width 0.2) (layer "F.Cu") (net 2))
 (segment (start 102.63 134.36) (end 105.29 131.7) (width 0.2) (layer "F.Cu") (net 2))
 (segment (start 117.579 110.98) (end 117.579 107.839) (width 0.2) (layer "F.Cu") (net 2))
 (segment (start 105.29 131.7) (end 105.29 123.269) (width 0.2) (layer "F.Cu") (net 2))
 (segment (start 117.579 107.839) (end 121.131 107.839) (width 0.2) (layer "F.Cu") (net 2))
 (segment (start 105.29 123.269) (end 117.579 110.98) (width 0.2) (layer "F.Cu") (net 2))
 (segment (start 166.58 104.548) (end 157.151 95.119) (width 0.2) (layer "F.Cu") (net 5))
 (segment (start 133.1468 87.376) (end 133.1468 100.5918) (width 0.2) (layer "F.Cu") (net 5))
 (segment (start 133.21 102.642) (end 135.197 102.642) (width 0.2) (layer "F.Cu") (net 5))
 (segment (start 120.21 115.93) (end 120.15 115.87) (width 0.2) (layer "F.Cu") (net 5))
 (segment (start 135.197 102.642) (end 135.482 102.642) (width 0.2) (layer "F.Cu") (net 5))
 (segment (start 131.12 108.585) (end 133.105 108.585) (width 0.2) (layer "F.Cu") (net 5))
 (segment (start 133.1722 87.376) (end 133.1976 87.3506) (width 0.2) (layer "F.Cu") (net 5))
 (segment (start 137.0223 87.3252) (end 139.491 89.7939) (width 0.2) (layer "F.Cu") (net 5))
 (segment (start 133.21 108.48) (end 133.21 102.642) (width 0.2) (layer "F.Cu") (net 5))
 (segment (start 123.835 115.87) (end 131.12 108.585) (width 0.2) (layer "F.Cu") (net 5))
 (segment (start 157.151 95.119) (end 155.049 95.119) (width 0.2) (layer "F.Cu") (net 5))
 (segment (start 148.5392 83.185) (end 148.5646 83.185) (width 0.2) (layer "F.Cu") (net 5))
 (segment (start 133.105 108.585) (end 133.21 108.48) (width 0.2) (layer "F.Cu") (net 5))
 (segment (start 148.5646 83.185) (end 148.59 83.2104) (width 0.2) (layer "F.Cu") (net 5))
 (segment (start 139.491 96.859) (end 147.709 88.641) (width 0.2) (layer "F.Cu") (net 5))
 (segment (start 170.75 115.96) (end 166.58 111.79) (width 0.2) (layer "F.Cu") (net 5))
 (segment (start 139.491 89.7939) (end 139.491 96.859) (width 0.2) (layer "F.Cu") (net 5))
 (segment (start 136.144 87.3252) (end 137.0223 87.3252) (width 0.2) (layer "F.Cu") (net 5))
 (segment (start 145.8722 80.518) (end 148.5392 83.185) (width 0.2) (layer "F.Cu") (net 5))
 (segment (start 147.828 86.9188) (end 147.828 88.522) (width 0.2) (layer "F.Cu") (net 5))
 (segment (start 147.828 88.522) (end 147.709 88.641) (width 0.2) (layer "F.Cu") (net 5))
 (segment (start 145.8722 68.9864) (end 145.8722 80.518) (width 0.2) (layer "F.Cu") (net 5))
 (segment (start 120.21 115.96) (end 120.21 115.93) (width 0.2) (layer "F.Cu") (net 5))
 (segment (start 152.576058 88.641) (end 147.709 88.641) (width 0.2) (layer "F.Cu") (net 5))
 (segment (start 135.482 102.642) (end 135.49 102.65) (width 0.2) (layer "F.Cu") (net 5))
 (segment (start 155.049 95.119) (end 155.049 91.113942) (width 0.2) (layer "F.Cu") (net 5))
 (segment (start 155.049 91.113942) (end 152.576058 88.641) (width 0.2) (layer "F.Cu") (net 5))
 (segment (start 145.71 69.23) (end 145.71 69.1486) (width 0.2) (layer "F.Cu") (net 5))
 (segment (start 120.15 115.87) (end 123.835 115.87) (width 0.2) (layer "F.Cu") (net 5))
 (segment (start 133.1468 87.376) (end 133.1722 87.376) (width 0.2) (layer "F.Cu") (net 5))
 (segment (start 145.71 69.1486) (end 145.8722 68.9864) (width 0.2) (layer "F.Cu") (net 5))
 (segment (start 133.1468 100.5918) (end 135.197 102.642) (width 0.2) (layer "F.Cu") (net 5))
 (segment (start 166.58 111.79) (end 166.58 104.548) (width 0.2) (layer "F.Cu") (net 5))
 (via (at 147.828 86.9188) (size 0.6) (drill 0.3) (layers "F.Cu" "B.Cu") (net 5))
 (via (at 136.144 87.3252) (size 0.6) (drill 0.3) (layers "F.Cu" "B.Cu") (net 5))
 (via (at 148.59 83.2104) (size 0.6) (drill 0.3) (layers "F.Cu" "B.Cu") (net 5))
 (via (at 133.1976 87.3506) (size 0.6) (drill 0.3) (layers "F.Cu" "B.Cu") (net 5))
 (segment (start 147.8534 86.8934) (end 147.828 86.9188) (width 0.2) (layer "B.Cu") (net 5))
 (segment (start 136.144 87.3252) (end 136.2456 87.3252) (width 0.2) (layer "B.Cu") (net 5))
 (segment (start 147.8534 86.868) (end 147.8534 86.8934) (width 0.2) (layer "B.Cu") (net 5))
 (segment (start 133.223 87.3252) (end 136.144 87.3252) (width 0.2) (layer "B.Cu") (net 5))
 (segment (start 147.8534 83.947) (end 147.8534 86.868) (width 0.2) (layer "B.Cu") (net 5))
 (segment (start 133.1976 87.3506) (end 133.223 87.3252) (width 0.2) (layer "B.Cu") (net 5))
 (segment (start 148.59 83.2104) (end 147.8534 83.947) (width 0.2) (layer "B.Cu") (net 5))
 (segment (start 143.95 94.58) (end 143.95 100.08) (width 0.2) (layer "F.Cu") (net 19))
 (segment (start 143.98 100.11) (end 143.988 100.102) (width 0.2) (layer "F.Cu") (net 19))
 (segment (start 143.95 100.08) (end 143.98 100.11) (width 0.2) (layer "F.Cu") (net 19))
 (segment (start 143.988 100.102) (end 151.362 100.102) (width 0.2) (layer "F.Cu") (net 19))
 (via (at 143.95 94.58) (size 0.6) (drill 0.3) (layers "F.Cu" "B.Cu") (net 19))
 (segment (start 139.36 91.11) (end 141.08 92.83) (width 0.2) (layer "B.Cu") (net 19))
 (segment (start 143.91 94.46) (end 143.95 94.5) (width 0.2) (layer "B.Cu") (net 19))
 (segment (start 143.91 94.28) (end 143.91 94.46) (width 0.2) (layer "B.Cu") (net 19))
 (segment (start 141.08 92.83) (end 142.46 92.83) (width 0.2) (layer "B.Cu") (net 19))
 (segment (start 142.46 92.83) (end 143.91 94.28) (width 0.2) (layer "B.Cu") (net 19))
 (segment (start 143.95 94.5) (end 143.95 94.58) (width 0.2) (layer "B.Cu") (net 19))
 (segment (start 139.36 71.77) (end 139.36 91.11) (width 0.2) (layer "B.Cu") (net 19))
 (segment (start 151.362 102.642) (end 160.054 102.642) (width 0.2) (layer "F.Cu") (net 6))
 (segment (start 160.054 102.642) (end 166.179 108.767) (width 0.2) (layer "F.Cu") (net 6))
 (segment (start 166.179 116.721) (end 166.179 108.767) (width 0.2) (layer "F.Cu") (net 6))
 (segment (start 164.4 118.5) (end 166.179 116.721) (width 0.2) (layer "F.Cu") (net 6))
 (segment (start 150.969 104.789) (end 151.362 105.182) (width 0.2) (layer "F.Cu") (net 18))
 (segment (start 132.940468 111.710468) (end 139.861936 104.789) (width 0.2) (layer "F.Cu") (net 18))
 (segment (start 126.150936 118.5) (end 132.940468 111.710468) (width 0.2) (layer "F.Cu") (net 18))
 (segment (start 139.861936 104.789) (end 150.969 104.789) (width 0.2) (layer "F.Cu") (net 18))
 (segment (start 113.86 118.5) (end 126.150936 118.5) (width 0.2) (layer "F.Cu") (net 18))
 (segment (start 136.158 100.102) (end 135.197 100.102) (width 0.2) (layer "F.Cu") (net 10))
 (segment (start 136.128229 106.765829) (end 136.873 106.021058) (width 0.2) (layer "F.Cu") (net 10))
 (segment (start 118.809 116.540314) (end 119.629686 117.361) (width 0.2) (layer "F.Cu") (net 10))
 (segment (start 136.873 106.021058) (end 136.873 101.778) (width 0.2) (layer "F.Cu") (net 10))
 (segment (start 119.629686 117.361) (end 125.533058 117.361) (width 0.2) (layer "F.Cu") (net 10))
 (segment (start 125.29 111.24) (end 125.29 111.1586) (width 0.2) (layer "F.Cu") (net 10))
 (segment (start 136.873 101.778) (end 135.197 100.102) (width 0.2) (layer "F.Cu") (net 10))
 (segment (start 119.629686 117.361) (end 125.730314 117.361) (width 0.2) (layer "F.Cu") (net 10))
 (segment (start 118.809 115.379686) (end 118.809 116.540314) (width 0.2) (layer "F.Cu") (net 10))
 (segment (start 125.29 111.1586) (end 125.3744 111.0742) (width 0.2) (layer "F.Cu") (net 10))
 (segment (start 125.3744 111.0742) (end 123.114486 111.0742) (width 0.2) (layer "F.Cu") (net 10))
 (segment (start 125.533058 117.361) (end 133.893029 109.001029) (width 0.2) (layer "F.Cu") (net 10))
 (segment (start 123.114486 111.0742) (end 118.809 115.379686) (width 0.2) (layer "F.Cu") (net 10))
 (via (at 136.128229 106.765829) (size 0.6) (drill 0.3) (layers "F.Cu" "B.Cu") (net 10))
 (via (at 133.893029 109.001029) (size 0.6) (drill 0.3) (layers "F.Cu" "B.Cu") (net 10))
 (segment (start 136.128229 106.765829) (end 135.480529 107.413529) (width 0.2) (layer "B.Cu") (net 10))
 (segment (start 135.480529 107.413529) (end 135.480529 107.445071) (width 0.2) (layer "B.Cu") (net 10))
 (segment (start 135.480529 107.445071) (end 133.924571 109.001029) (width 0.2) (layer "B.Cu") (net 10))
 (segment (start 133.924571 109.001029) (end 133.893029 109.001029) (width 0.2) (layer "B.Cu") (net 10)))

